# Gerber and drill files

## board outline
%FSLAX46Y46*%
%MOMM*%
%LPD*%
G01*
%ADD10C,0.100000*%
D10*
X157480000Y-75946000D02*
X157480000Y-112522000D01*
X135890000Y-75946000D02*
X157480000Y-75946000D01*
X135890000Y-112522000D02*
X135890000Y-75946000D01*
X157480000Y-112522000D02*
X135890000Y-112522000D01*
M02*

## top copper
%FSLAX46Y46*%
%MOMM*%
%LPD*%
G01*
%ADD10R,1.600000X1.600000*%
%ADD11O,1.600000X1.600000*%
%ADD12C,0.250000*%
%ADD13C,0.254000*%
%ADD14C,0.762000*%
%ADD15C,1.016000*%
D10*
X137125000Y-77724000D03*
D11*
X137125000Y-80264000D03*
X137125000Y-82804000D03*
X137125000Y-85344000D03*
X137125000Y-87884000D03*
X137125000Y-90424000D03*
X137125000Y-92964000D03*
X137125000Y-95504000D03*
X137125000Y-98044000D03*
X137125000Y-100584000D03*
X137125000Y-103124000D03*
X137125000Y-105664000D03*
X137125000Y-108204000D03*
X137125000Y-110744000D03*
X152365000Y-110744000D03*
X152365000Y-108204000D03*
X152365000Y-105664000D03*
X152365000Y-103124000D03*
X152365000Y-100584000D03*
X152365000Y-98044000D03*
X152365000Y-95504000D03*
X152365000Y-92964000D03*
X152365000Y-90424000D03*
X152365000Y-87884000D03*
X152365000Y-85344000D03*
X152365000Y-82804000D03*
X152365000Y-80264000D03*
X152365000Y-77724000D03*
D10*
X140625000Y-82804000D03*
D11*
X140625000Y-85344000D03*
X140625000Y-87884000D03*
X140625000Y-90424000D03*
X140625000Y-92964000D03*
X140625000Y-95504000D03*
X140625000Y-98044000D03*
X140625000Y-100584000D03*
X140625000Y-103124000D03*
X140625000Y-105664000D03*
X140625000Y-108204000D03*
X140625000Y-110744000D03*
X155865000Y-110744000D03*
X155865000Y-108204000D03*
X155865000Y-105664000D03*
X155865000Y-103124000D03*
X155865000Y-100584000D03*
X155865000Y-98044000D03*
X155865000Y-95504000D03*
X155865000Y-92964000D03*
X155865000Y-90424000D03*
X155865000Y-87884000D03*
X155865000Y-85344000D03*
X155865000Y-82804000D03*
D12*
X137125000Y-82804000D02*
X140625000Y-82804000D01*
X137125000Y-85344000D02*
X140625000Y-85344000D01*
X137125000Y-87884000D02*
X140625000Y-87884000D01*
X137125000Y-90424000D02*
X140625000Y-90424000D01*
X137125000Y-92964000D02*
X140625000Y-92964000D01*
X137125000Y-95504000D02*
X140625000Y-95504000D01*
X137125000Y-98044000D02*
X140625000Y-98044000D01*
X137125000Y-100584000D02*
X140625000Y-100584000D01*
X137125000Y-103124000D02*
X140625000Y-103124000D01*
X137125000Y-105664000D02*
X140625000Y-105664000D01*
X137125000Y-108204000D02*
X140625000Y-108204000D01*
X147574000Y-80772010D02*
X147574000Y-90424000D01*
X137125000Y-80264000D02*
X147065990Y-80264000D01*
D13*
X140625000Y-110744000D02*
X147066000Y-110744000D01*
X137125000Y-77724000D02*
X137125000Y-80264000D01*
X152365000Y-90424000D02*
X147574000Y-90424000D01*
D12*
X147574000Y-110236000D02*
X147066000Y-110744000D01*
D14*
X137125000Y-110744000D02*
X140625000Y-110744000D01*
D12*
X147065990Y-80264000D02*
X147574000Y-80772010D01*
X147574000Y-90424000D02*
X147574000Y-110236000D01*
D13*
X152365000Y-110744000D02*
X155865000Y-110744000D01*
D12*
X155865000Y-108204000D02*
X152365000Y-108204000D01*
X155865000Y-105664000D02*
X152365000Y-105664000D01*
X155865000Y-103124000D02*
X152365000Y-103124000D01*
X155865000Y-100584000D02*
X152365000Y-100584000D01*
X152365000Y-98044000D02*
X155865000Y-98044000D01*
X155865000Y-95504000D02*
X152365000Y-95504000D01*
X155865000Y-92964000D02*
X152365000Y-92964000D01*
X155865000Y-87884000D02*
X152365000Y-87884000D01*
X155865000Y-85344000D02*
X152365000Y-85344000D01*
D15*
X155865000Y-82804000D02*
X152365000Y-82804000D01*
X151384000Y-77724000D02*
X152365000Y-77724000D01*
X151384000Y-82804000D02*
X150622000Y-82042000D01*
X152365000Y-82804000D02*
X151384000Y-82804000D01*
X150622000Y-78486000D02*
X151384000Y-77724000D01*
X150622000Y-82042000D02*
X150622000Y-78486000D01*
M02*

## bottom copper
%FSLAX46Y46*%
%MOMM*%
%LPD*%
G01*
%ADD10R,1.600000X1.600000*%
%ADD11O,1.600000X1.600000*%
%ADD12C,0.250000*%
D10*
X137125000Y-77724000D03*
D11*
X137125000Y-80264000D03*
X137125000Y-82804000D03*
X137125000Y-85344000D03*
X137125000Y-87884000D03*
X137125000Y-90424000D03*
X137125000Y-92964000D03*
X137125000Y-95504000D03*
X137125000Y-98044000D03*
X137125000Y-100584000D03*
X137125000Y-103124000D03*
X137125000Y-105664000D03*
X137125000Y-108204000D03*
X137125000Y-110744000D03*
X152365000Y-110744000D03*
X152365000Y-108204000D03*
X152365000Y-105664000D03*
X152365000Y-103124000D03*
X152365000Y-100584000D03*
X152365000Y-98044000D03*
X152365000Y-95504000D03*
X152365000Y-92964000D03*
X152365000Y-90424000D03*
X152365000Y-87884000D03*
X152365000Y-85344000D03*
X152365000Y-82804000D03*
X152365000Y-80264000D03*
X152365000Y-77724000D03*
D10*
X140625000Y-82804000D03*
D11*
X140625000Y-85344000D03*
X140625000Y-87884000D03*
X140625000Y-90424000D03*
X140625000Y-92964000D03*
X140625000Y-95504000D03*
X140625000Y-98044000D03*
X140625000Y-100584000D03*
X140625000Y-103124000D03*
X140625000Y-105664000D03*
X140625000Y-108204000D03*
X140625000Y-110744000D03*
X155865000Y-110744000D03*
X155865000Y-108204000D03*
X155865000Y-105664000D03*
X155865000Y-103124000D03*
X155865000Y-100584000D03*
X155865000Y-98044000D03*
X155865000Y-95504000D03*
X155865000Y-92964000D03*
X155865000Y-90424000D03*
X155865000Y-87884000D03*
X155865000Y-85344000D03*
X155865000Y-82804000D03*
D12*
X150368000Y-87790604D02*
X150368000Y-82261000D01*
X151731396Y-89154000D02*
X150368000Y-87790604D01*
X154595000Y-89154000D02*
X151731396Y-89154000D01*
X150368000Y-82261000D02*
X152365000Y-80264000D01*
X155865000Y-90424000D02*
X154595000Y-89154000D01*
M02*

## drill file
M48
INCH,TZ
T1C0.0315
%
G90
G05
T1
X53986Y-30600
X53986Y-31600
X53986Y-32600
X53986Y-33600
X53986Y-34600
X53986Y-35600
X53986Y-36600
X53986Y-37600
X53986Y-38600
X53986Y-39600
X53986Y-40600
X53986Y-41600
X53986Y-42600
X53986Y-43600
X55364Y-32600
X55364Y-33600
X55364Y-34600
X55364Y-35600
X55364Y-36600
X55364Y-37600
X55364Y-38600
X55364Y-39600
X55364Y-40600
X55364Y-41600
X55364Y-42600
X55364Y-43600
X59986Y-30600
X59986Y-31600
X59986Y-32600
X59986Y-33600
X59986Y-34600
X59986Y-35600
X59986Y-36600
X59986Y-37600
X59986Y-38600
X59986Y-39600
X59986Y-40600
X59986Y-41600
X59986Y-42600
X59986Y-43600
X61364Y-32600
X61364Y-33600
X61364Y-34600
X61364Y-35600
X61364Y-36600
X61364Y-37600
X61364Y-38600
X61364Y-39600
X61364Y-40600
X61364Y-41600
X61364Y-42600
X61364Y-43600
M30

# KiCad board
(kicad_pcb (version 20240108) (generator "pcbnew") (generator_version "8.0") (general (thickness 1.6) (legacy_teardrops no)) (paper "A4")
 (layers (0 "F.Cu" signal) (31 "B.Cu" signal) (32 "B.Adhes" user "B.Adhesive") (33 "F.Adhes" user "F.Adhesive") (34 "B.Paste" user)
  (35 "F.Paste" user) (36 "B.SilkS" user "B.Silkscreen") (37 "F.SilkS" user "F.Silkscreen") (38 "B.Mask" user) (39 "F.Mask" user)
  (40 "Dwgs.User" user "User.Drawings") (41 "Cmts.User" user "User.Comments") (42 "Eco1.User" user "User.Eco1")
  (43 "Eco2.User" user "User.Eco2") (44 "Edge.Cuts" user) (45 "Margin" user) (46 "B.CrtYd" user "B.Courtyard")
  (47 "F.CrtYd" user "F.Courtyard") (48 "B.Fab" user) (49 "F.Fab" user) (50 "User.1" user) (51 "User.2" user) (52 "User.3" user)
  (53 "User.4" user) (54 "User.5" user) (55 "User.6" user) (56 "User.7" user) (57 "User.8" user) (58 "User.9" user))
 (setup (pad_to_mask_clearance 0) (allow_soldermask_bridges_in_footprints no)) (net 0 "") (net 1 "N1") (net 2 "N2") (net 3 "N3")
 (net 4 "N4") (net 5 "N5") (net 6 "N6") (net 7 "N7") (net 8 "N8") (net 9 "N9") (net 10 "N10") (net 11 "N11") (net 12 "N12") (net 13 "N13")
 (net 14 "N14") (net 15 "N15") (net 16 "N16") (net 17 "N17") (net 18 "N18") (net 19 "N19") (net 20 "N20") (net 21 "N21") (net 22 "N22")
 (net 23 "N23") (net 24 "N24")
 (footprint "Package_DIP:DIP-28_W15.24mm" (layer "F.Cu") (at 137.125 77.724)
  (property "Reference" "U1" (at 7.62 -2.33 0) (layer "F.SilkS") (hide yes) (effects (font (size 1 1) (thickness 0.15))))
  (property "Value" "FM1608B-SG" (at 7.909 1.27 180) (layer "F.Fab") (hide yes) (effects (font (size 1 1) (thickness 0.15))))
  (pad "1" thru_hole rect (at 0 0) (size 1.6 1.6) (drill 0.8) (layers "*.Cu" "*.Mask") (remove_unused_layers no) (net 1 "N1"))
  (pad "2" thru_hole oval (at 0 2.54) (size 1.6 1.6) (drill 0.8) (layers "*.Cu" "*.Mask") (remove_unused_layers no) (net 1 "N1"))
  (pad "3" thru_hole oval (at 0 5.08) (size 1.6 1.6) (drill 0.8) (layers "*.Cu" "*.Mask") (remove_unused_layers no) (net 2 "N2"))
  (pad "4" thru_hole oval (at 0 7.62) (size 1.6 1.6) (drill 0.8) (layers "*.Cu" "*.Mask") (remove_unused_layers no) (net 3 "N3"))
  (pad "5" thru_hole oval (at 0 10.16) (size 1.6 1.6) (drill 0.8) (layers "*.Cu" "*.Mask") (remove_unused_layers no) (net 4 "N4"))
  (pad "6" thru_hole oval (at 0 12.7) (size 1.6 1.6) (drill 0.8) (layers "*.Cu" "*.Mask") (remove_unused_layers no) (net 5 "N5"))
  (pad "7" thru_hole oval (at 0 15.24) (size 1.6 1.6) (drill 0.8) (layers "*.Cu" "*.Mask") (remove_unused_layers no) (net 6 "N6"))
  (pad "8" thru_hole oval (at 0 17.78) (size 1.6 1.6) (drill 0.8) (layers "*.Cu" "*.Mask") (remove_unused_layers no) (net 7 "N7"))
  (pad "9" thru_hole oval (at 0 20.32) (size 1.6 1.6) (drill 0.8) (layers "*.Cu" "*.Mask") (remove_unused_layers no) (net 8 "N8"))
  (pad "10" thru_hole oval (at 0 22.86) (size 1.6 1.6) (drill 0.8) (layers "*.Cu" "*.Mask") (remove_unused_layers no) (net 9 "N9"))
  (pad "11" thru_hole oval (at 0 25.4) (size 1.6 1.6) (drill 0.8) (layers "*.Cu" "*.Mask") (remove_unused_layers no) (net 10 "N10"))
  (pad "12" thru_hole oval (at 0 27.94) (size 1.6 1.6) (drill 0.8) (layers "*.Cu" "*.Mask") (remove_unused_layers no) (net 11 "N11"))
  (pad "13" thru_hole oval (at 0 30.48) (size 1.6 1.6) (drill 0.8) (layers "*.Cu" "*.Mask") (remove_unused_layers no) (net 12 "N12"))
  (pad "14" thru_hole oval (at 0 33.02) (size 1.6 1.6) (drill 0.8) (layers "*.Cu" "*.Mask") (remove_unused_layers no) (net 1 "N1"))
  (pad "15" thru_hole oval (at 15.24 33.02) (size 1.6 1.6) (drill 0.8) (layers "*.Cu" "*.Mask") (remove_unused_layers no) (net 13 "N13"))
  (pad "16" thru_hole oval (at 15.24 30.48) (size 1.6 1.6) (drill 0.8) (layers "*.Cu" "*.Mask") (remove_unused_layers no) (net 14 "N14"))
  (pad "17" thru_hole oval (at 15.24 27.94) (size 1.6 1.6) (drill 0.8) (layers "*.Cu" "*.Mask") (remove_unused_layers no) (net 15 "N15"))
  (pad "18" thru_hole oval (at 15.24 25.4) (size 1.6 1.6) (drill 0.8) (layers "*.Cu" "*.Mask") (remove_unused_layers no) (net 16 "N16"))
  (pad "19" thru_hole oval (at 15.24 22.86) (size 1.6 1.6) (drill 0.8) (layers "*.Cu" "*.Mask") (remove_unused_layers no) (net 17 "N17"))
  (pad "20" thru_hole oval (at 15.24 20.32) (size 1.6 1.6) (drill 0.8) (layers "*.Cu" "*.Mask") (remove_unused_layers no) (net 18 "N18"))
  (pad "21" thru_hole oval (at 15.24 17.78) (size 1.6 1.6) (drill 0.8) (layers "*.Cu" "*.Mask") (remove_unused_layers no) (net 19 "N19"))
  (pad "22" thru_hole oval (at 15.24 15.24) (size 1.6 1.6) (drill 0.8) (layers "*.Cu" "*.Mask") (remove_unused_layers no) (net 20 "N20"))
  (pad "23" thru_hole oval (at 15.24 12.7) (size 1.6 1.6) (drill 0.8) (layers "*.Cu" "*.Mask") (remove_unused_layers no) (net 1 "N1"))
  (pad "24" thru_hole oval (at 15.24 10.16) (size 1.6 1.6) (drill 0.8) (layers "*.Cu" "*.Mask") (remove_unused_layers no) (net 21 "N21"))
  (pad "25" thru_hole oval (at 15.24 7.62) (size 1.6 1.6) (drill 0.8) (layers "*.Cu" "*.Mask") (remove_unused_layers no) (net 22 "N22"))
  (pad "26" thru_hole oval (at 15.24 5.08) (size 1.6 1.6) (drill 0.8) (layers "*.Cu" "*.Mask") (remove_unused_layers no) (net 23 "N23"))
  (pad "27" thru_hole oval (at 15.24 2.54) (size 1.6 1.6) (drill 0.8) (layers "*.Cu" "*.Mask") (remove_unused_layers no) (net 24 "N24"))
  (pad "28" thru_hole oval (at 15.24 0) (size 1.6 1.6) (drill 0.8) (layers "*.Cu" "*.Mask") (remove_unused_layers no) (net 23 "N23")))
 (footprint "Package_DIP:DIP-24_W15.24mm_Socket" (layer "F.Cu") (at 140.625 82.804)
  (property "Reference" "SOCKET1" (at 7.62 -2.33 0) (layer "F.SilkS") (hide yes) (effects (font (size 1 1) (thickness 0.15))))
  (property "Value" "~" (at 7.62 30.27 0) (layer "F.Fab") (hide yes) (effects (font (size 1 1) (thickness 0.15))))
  (pad "1" thru_hole rect (at 0 0) (size 1.6 1.6) (drill 0.8) (layers "*.Cu" "*.Mask") (remove_unused_layers no) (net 2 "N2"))
  (pad "2" thru_hole oval (at 0 2.54) (size 1.6 1.6) (drill 0.8) (layers "*.Cu" "*.Mask") (remove_unused_layers no) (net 3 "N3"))
  (pad "3" thru_hole oval (at 0 5.08) (size 1.6 1.6) (drill 0.8) (layers "*.Cu" "*.Mask") (remove_unused_layers no) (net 4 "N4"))
  (pad "4" thru_hole oval (at 0 7.62) (size 1.6 1.6) (drill 0.8) (layers "*.Cu" "*.Mask") (remove_unused_layers no) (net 5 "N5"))
  (pad "5" thru_hole oval (at 0 10.16) (size 1.6 1.6) (drill 0.8) (layers "*.Cu" "*.Mask") (remove_unused_layers no) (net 6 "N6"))
  (pad "6" thru_hole oval (at 0 12.7) (size 1.6 1.6) (drill 0.8) (layers "*.Cu" "*.Mask") (remove_unused_layers no) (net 7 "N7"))
  (pad "7" thru_hole oval (at 0 15.24) (size 1.6 1.6) (drill 0.8) (layers "*.Cu" "*.Mask") (remove_unused_layers no) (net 8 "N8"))
  (pad "8" thru_hole oval (at 0 17.78) (size 1.6 1.6) (drill 0.8) (layers "*.Cu" "*.Mask") (remove_unused_layers no) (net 9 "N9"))
  (pad "9" thru_hole oval (at 0 20.32) (size 1.6 1.6) (drill 0.8) (layers "*.Cu" "*.Mask") (remove_unused_layers no) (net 10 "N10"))
  (pad "10" thru_hole oval (at 0 22.86) (size 1.6 1.6) (drill 0.8) (layers "*.Cu" "*.Mask") (remove_unused_layers no) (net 11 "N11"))
  (pad "11" thru_hole oval (at 0 25.4) (size 1.6 1.6) (drill 0.8) (layers "*.Cu" "*.Mask") (remove_unused_layers no) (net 12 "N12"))
  (pad "12" thru_hole oval (at 0 27.94) (size 1.6 1.6) (drill 0.8) (layers "*.Cu" "*.Mask") (remove_unused_layers no) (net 1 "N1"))
  (pad "13" thru_hole oval (at 15.24 27.94) (size 1.6 1.6) (drill 0.8) (layers "*.Cu" "*.Mask") (remove_unused_layers no) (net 13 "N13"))
  (pad "14" thru_hole oval (at 15.24 25.4) (size 1.6 1.6) (drill 0.8) (layers "*.Cu" "*.Mask") (remove_unused_layers no) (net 14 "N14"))
  (pad "15" thru_hole oval (at 15.24 22.86) (size 1.6 1.6) (drill 0.8) (layers "*.Cu" "*.Mask") (remove_unused_layers no) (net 15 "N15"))
  (pad "16" thru_hole oval (at 15.24 20.32) (size 1.6 1.6) (drill 0.8) (layers "*.Cu" "*.Mask") (remove_unused_layers no) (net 16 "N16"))
  (pad "17" thru_hole oval (at 15.24 17.78) (size 1.6 1.6) (drill 0.8) (layers "*.Cu" "*.Mask") (remove_unused_layers no) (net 17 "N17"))
  (pad "18" thru_hole oval (at 15.24 15.24) (size 1.6 1.6) (drill 0.8) (layers "*.Cu" "*.Mask") (remove_unused_layers no) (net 18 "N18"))
  (pad "19" thru_hole oval (at 15.24 12.7) (size 1.6 1.6) (drill 0.8) (layers "*.Cu" "*.Mask") (remove_unused_layers no) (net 19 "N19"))
  (pad "20" thru_hole oval (at 15.24 10.16) (size 1.6 1.6) (drill 0.8) (layers "*.Cu" "*.Mask") (remove_unused_layers no) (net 20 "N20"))
  (pad "21" thru_hole oval (at 15.24 7.62) (size 1.6 1.6) (drill 0.8) (layers "*.Cu" "*.Mask") (remove_unused_layers no) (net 24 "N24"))
  (pad "22" thru_hole oval (at 15.24 5.08) (size 1.6 1.6) (drill 0.8) (layers "*.Cu" "*.Mask") (remove_unused_layers no) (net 21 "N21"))
  (pad "23" thru_hole oval (at 15.24 2.54) (size 1.6 1.6) (drill 0.8) (layers "*.Cu" "*.Mask") (remove_unused_layers no) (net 22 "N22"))
  (pad "24" thru_hole oval (at 15.24 0) (size 1.6 1.6) (drill 0.8) (layers "*.Cu" "*.Mask") (remove_unused_layers no) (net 23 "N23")))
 (gr_line (start 157.48 75.946) (end 157.48 112.522) (stroke (width 0.1) (type default)) (layer "Edge.Cuts"))
 (gr_line (start 135.89 75.946) (end 157.48 75.946) (stroke (width 0.1) (type default)) (layer "Edge.Cuts"))
 (gr_line (start 135.89 112.522) (end 135.89 75.946) (stroke (width 0.1) (type default)) (layer "Edge.Cuts"))
 (gr_line (start 157.48 112.522) (end 135.89 112.522) (stroke (width 0.1) (type default)) (layer "Edge.Cuts"))
 (segment (start 137.125 82.804) (end 140.625 82.804) (width 0.25) (layer "F.Cu") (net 2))
 (segment (start 137.125 85.344) (end 140.625 85.344) (width 0.25) (layer "F.Cu") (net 3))
 (segment (start 137.125 87.884) (end 140.625 87.884) (width 0.25) (layer "F.Cu") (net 4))
 (segment (start 137.125 90.424) (end 140.625 90.424) (width 0.25) (layer "F.Cu") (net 5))
 (segment (start 137.125 92.964) (end 140.625 92.964) (width 0.25) (layer "F.Cu") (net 6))
 (segment (start 137.125 95.504) (end 140.625 95.504) (width 0.25) (layer "F.Cu") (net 7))
 (segment (start 137.125 98.044) (end 140.625 98.044) (width 0.25) (layer "F.Cu") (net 8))
 (segment (start 137.125 100.584) (end 140.625 100.584) (width 0.25) (layer "F.Cu") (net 9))
 (segment (start 137.125 103.124) (end 140.625 103.124) (width 0.25) (layer "F.Cu") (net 10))
 (segment (start 137.125 105.664) (end 140.625 105.664) (width 0.25) (layer "F.Cu") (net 11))
 (segment (start 137.125 108.204) (end 140.625 108.204) (width 0.25) (layer "F.Cu") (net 12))
 (segment (start 147.574 80.77201) (end 147.574 90.424) (width 0.25) (layer "F.Cu") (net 1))
 (segment (start 137.125 80.264) (end 147.06599 80.264) (width 0.25) (layer "F.Cu") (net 1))
 (segment (start 140.625 110.744) (end 147.066 110.744) (width 0.254) (layer "F.Cu") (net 1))
 (segment (start 137.125 77.724) (end 137.125 80.264) (width 0.254) (layer "F.Cu") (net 1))
 (segment (start 152.365 90.424) (end 147.574 90.424) (width 0.254) (layer "F.Cu") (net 1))
 (segment (start 147.574 110.236) (end 147.066 110.744) (width 0.25) (layer "F.Cu") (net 1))
 (segment (start 137.125 110.744) (end 140.625 110.744) (width 0.762) (layer "F.Cu") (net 1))
 (segment (start 147.06599 80.264) (end 147.574 80.77201) (width 0.25) (layer "F.Cu") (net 1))
 (segment (start 147.574 90.424) (end 147.574 110.236) (width 0.25) (layer "F.Cu") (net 1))
 (segment (start 152.365 110.744) (end 155.865 110.744) (width 0.254) (layer "F.Cu") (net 13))
 (segment (start 155.865 108.204) (end 152.365 108.204) (width 0.25) (layer "F.Cu") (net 14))
 (segment (start 155.865 105.664) (end 152.365 105.664) (width 0.25) (layer "F.Cu") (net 15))
 (segment (start 155.865 103.124) (end 152.365 103.124) (width 0.25) (layer "F.Cu") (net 16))
 (segment (start 155.865 100.584) (end 152.365 100.584) (width 0.25) (layer "F.Cu") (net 17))
 (segment (start 152.365 98.044) (end 155.865 98.044) (width 0.25) (layer "F.Cu") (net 18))
 (segment (start 155.865 95.504) (end 152.365 95.504) (width 0.25) (layer "F.Cu") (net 19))
 (segment (start 155.865 92.964) (end 152.365 92.964) (width 0.25) (layer "F.Cu") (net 20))
 (segment (start 150.368 87.790604) (end 150.368 82.261) (width 0.25) (layer "B.Cu") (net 24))
 (segment (start 151.731396 89.154) (end 150.368 87.790604) (width 0.25) (layer "B.Cu") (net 24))
 (segment (start 154.595 89.154) (end 151.731396 89.154) (width 0.25) (layer "B.Cu") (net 24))
 (segment (start 150.368 82.261) (end 152.365 80.264) (width 0.25) (layer "B.Cu") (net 24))
 (segment (start 155.865 90.424) (end 154.595 89.154) (width 0.25) (layer "B.Cu") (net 24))
 (segment (start 155.865 87.884) (end 152.365 87.884) (width 0.25) (layer "F.Cu") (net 21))
 (segment (start 155.865 85.344) (end 152.365 85.344) (width 0.25) (layer "F.Cu") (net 22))
 (segment (start 155.865 82.804) (end 152.365 82.804) (width 1.016) (layer "F.Cu") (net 23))
 (segment (start 151.384 77.724) (end 152.365 77.724) (width 1.016) (layer "F.Cu") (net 23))
 (segment (start 151.384 82.804) (end 150.622 82.042) (width 1.016) (layer "F.Cu") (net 23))
 (segment (start 152.365 82.804) (end 151.384 82.804) (width 1.016) (layer "F.Cu") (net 23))
 (segment (start 150.622 78.486) (end 151.384 77.724) (width 1.016) (layer "F.Cu") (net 23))
 (segment (start 150.622 82.042) (end 150.622 78.486) (width 1.016) (layer "F.Cu") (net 23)))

